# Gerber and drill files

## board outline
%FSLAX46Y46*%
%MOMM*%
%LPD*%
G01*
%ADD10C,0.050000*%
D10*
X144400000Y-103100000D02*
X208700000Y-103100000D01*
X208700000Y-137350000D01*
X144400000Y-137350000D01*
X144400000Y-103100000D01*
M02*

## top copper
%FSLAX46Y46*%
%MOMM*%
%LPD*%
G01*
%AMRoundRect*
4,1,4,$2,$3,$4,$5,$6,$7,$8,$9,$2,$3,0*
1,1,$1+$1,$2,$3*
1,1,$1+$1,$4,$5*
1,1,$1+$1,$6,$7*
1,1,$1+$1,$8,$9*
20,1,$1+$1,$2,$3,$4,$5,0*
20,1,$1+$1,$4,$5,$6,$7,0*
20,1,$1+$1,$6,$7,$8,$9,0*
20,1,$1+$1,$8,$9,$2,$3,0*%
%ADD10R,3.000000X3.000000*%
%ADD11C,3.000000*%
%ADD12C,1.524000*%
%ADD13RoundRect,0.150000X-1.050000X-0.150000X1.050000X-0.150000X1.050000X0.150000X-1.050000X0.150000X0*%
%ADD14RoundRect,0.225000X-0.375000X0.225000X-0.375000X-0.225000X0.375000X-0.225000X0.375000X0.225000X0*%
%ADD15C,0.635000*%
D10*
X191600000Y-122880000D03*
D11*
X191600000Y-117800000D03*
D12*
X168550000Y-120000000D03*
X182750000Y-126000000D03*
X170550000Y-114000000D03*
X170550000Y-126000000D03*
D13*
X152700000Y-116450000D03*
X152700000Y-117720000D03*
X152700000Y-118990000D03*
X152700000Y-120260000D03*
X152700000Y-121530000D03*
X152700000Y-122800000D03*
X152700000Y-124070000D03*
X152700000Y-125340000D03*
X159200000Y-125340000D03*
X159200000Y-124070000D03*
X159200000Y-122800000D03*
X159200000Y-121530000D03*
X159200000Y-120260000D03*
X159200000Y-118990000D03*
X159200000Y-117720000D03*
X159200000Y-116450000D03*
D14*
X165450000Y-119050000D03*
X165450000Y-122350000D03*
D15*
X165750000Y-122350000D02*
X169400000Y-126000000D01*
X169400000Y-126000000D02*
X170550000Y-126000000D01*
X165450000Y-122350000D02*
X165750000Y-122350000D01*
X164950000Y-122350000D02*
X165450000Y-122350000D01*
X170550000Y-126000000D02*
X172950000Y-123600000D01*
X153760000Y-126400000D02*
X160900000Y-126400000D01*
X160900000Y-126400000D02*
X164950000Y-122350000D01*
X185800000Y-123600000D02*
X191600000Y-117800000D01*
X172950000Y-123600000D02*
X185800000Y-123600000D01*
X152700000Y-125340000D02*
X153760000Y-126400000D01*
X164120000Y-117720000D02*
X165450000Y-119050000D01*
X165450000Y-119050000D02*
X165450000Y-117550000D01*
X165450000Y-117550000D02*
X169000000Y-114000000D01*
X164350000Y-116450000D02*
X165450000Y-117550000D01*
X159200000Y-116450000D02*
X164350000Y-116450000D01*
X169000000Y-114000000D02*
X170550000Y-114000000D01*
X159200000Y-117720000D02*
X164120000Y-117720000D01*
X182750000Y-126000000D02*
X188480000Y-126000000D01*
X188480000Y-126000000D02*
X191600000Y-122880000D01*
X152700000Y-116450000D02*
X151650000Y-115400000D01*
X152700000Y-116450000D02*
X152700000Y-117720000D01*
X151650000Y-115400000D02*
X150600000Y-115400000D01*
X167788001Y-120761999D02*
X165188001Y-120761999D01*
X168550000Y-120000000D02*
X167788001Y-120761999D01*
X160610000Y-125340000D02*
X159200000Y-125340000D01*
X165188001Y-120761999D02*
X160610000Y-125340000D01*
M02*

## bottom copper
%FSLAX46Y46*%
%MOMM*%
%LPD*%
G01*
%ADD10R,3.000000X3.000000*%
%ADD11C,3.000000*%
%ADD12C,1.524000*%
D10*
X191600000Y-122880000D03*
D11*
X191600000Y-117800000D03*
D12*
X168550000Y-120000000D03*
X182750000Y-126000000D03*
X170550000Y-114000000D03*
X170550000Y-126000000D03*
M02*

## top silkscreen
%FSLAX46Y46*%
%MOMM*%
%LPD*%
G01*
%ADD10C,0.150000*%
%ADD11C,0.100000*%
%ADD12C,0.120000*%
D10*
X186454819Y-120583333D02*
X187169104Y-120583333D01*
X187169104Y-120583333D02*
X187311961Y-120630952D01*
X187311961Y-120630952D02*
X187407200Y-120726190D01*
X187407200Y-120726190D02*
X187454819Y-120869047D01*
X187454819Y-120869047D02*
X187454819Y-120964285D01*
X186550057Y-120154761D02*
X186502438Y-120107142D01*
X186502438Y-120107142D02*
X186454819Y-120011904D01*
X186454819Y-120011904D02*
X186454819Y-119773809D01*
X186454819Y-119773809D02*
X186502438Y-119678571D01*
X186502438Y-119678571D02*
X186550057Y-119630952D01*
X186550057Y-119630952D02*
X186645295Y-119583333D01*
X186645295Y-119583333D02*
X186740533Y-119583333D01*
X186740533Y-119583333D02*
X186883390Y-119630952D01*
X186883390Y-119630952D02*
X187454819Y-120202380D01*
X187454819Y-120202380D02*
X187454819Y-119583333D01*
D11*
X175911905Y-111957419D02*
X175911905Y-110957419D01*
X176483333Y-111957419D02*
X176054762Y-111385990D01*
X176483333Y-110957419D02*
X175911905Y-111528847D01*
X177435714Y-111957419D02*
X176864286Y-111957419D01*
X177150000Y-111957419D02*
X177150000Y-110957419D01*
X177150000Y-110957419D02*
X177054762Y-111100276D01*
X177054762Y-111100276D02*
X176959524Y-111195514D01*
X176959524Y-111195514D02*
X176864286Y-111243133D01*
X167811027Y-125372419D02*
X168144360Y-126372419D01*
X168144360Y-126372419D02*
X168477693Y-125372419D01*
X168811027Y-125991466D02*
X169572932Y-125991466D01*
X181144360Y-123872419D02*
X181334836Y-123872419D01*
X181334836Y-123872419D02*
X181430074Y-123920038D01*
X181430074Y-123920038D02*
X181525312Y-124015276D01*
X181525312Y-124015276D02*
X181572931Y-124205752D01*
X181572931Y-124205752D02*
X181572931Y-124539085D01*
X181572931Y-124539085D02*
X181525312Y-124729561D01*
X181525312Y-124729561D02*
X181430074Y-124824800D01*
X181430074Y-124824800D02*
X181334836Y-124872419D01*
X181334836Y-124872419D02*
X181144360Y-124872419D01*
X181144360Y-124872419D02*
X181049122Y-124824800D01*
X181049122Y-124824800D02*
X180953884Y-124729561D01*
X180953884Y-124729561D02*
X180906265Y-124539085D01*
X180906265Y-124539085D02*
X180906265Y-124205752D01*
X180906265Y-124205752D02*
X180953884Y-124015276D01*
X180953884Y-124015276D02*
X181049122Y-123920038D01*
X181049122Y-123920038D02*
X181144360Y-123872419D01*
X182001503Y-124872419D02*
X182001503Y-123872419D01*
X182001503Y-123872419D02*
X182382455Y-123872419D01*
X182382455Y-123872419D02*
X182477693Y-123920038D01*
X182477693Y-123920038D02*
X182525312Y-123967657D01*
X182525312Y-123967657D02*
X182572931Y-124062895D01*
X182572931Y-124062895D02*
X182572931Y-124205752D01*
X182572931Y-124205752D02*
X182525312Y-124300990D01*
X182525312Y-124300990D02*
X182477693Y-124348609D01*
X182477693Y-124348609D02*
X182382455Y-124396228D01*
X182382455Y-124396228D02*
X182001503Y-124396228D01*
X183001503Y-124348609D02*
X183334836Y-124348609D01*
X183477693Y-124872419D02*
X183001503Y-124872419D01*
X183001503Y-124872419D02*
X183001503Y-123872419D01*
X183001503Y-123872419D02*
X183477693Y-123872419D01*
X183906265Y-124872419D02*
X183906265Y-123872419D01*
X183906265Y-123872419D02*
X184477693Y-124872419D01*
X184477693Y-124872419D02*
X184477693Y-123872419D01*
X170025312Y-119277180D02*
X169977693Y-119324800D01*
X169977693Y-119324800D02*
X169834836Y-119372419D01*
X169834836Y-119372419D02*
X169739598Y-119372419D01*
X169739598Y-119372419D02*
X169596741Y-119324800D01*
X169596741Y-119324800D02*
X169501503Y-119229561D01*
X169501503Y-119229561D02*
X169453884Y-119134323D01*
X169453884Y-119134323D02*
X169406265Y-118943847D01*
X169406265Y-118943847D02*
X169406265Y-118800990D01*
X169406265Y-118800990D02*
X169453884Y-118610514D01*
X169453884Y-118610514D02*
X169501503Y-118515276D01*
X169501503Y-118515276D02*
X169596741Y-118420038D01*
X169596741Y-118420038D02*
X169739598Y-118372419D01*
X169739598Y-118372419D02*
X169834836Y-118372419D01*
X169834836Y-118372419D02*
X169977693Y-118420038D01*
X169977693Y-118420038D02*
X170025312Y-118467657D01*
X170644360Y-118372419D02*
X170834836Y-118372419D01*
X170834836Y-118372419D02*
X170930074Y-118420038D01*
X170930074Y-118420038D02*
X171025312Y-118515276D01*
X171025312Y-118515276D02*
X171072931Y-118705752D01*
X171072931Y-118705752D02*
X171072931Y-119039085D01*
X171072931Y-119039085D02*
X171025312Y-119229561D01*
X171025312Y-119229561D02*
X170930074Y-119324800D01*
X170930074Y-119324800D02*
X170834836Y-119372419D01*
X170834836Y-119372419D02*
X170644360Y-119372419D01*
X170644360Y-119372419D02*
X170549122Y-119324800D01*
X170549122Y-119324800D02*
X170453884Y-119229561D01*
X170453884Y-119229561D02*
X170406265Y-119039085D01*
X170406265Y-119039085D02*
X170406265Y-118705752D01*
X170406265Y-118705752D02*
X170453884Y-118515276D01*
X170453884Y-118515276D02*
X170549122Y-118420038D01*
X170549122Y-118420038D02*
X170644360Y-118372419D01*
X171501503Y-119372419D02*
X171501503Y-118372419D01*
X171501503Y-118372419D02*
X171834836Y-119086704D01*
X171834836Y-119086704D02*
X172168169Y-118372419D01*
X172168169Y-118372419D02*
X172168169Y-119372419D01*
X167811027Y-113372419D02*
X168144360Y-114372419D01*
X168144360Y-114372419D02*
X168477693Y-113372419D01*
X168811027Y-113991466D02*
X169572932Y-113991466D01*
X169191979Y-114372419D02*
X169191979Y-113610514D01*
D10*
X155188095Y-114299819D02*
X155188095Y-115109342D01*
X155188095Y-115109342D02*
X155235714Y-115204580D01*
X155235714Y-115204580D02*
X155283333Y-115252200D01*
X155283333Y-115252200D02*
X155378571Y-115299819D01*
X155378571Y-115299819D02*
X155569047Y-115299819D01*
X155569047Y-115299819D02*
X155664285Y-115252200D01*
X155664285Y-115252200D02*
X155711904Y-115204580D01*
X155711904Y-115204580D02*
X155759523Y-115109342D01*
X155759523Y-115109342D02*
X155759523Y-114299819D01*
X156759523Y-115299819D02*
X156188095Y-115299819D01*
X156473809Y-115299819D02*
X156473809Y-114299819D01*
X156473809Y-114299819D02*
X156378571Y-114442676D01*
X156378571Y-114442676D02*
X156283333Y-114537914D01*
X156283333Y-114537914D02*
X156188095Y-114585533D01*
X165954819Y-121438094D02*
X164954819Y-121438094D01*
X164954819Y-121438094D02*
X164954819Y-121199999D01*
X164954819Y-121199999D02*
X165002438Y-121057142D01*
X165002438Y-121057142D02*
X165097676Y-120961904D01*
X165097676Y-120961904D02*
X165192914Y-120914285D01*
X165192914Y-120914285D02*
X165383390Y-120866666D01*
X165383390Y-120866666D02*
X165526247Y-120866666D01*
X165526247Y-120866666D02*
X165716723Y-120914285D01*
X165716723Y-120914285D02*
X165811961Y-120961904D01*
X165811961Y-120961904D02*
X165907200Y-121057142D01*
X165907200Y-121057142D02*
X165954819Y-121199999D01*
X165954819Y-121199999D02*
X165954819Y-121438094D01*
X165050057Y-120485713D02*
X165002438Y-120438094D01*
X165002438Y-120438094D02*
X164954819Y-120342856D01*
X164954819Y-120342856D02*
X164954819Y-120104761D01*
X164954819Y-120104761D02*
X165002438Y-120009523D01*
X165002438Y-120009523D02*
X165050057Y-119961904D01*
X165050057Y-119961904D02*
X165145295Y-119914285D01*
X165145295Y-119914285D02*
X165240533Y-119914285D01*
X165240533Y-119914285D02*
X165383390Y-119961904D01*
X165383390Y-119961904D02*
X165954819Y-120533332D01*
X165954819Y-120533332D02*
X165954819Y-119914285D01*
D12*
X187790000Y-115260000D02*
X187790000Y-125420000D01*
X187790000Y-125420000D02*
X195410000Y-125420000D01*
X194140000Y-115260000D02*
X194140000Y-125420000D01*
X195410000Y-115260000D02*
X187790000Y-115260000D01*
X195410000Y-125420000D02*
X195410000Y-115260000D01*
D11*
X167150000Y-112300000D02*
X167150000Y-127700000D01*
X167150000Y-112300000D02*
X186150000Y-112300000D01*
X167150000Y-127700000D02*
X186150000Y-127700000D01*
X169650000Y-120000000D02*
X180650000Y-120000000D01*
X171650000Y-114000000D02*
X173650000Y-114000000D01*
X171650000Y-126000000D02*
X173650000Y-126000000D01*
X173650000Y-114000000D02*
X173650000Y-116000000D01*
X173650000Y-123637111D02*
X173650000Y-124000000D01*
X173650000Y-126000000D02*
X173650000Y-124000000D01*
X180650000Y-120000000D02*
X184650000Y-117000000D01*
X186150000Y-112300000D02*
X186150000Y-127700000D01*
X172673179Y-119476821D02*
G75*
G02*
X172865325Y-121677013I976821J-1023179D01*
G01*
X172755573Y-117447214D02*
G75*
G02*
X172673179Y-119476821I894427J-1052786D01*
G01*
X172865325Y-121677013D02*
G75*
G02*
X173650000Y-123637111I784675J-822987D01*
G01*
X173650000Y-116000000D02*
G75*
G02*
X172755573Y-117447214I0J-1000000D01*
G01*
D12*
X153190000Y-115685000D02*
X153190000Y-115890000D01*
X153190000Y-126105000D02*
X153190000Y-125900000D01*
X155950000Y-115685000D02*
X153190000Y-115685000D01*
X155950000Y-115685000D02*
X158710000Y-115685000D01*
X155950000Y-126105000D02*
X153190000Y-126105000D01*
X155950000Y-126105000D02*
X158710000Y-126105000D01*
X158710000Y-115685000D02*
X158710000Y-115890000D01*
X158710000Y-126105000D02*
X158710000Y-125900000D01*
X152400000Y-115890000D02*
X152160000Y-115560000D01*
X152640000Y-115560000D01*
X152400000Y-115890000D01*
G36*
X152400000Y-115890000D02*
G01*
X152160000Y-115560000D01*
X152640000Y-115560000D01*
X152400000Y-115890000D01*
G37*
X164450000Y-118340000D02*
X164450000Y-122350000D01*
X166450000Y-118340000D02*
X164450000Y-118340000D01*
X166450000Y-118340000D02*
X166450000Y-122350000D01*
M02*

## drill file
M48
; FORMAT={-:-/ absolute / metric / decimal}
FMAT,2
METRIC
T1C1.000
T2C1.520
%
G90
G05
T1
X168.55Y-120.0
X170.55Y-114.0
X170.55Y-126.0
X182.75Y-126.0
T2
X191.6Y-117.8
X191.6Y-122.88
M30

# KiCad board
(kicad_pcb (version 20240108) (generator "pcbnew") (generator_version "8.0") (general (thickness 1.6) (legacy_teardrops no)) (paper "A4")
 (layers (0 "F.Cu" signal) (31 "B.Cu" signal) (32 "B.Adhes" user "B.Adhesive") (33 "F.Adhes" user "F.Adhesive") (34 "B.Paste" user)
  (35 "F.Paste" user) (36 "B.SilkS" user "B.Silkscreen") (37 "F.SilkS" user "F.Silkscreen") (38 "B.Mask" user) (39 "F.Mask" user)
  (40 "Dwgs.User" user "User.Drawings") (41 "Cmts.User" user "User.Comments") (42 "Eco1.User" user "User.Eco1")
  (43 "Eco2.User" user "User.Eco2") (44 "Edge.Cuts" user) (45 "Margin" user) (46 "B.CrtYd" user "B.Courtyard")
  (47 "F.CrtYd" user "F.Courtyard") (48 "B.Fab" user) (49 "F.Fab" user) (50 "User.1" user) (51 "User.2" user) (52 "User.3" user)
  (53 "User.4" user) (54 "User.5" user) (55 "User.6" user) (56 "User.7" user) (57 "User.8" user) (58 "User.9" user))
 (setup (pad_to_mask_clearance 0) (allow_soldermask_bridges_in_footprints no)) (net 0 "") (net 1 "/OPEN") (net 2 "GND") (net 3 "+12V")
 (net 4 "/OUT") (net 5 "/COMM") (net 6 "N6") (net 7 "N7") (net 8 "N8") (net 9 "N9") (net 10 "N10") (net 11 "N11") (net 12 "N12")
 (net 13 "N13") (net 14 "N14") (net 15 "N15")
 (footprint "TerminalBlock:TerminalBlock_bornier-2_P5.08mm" (layer "F.Cu") (at 191.6 122.88 90)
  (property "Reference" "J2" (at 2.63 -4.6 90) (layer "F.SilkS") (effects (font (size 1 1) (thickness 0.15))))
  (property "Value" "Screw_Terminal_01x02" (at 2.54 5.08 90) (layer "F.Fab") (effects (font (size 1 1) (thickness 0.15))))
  (fp_line (start 7.62 -3.81) (end -2.54 -3.81) (stroke (width 0.12) (type solid)) (layer "F.SilkS"))
  (fp_line (start -2.54 -3.81) (end -2.54 3.81) (stroke (width 0.12) (type solid)) (layer "F.SilkS"))
  (fp_line (start 7.62 2.54) (end -2.54 2.54) (stroke (width 0.12) (type solid)) (layer "F.SilkS"))
  (fp_line (start 7.62 3.81) (end 7.62 -3.81) (stroke (width 0.12) (type solid)) (layer "F.SilkS"))
  (fp_line (start -2.54 3.81) (end 7.62 3.81) (stroke (width 0.12) (type solid)) (layer "F.SilkS"))
  (pad "1" thru_hole rect (at 0 0 90) (size 3 3) (drill 1.52) (layers "*.Cu" "*.Mask") (remove_unused_layers no) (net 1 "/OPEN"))
  (pad "2" thru_hole circle (at 5.08 0 90) (size 3 3) (drill 1.52) (layers "*.Cu" "*.Mask") (remove_unused_layers no) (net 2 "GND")))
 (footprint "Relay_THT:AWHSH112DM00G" (layer "F.Cu") (at 176.65 120)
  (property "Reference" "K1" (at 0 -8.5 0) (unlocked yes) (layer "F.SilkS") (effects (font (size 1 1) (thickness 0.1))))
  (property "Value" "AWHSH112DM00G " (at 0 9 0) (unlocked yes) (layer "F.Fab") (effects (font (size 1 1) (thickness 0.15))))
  (fp_line (start -9.5 -7.7) (end -9.5 7.7) (stroke (width 0.1) (type default)) (layer "F.SilkS"))
  (fp_line (start -9.5 -7.7) (end 9.5 -7.7) (stroke (width 0.1) (type default)) (layer "F.SilkS"))
  (fp_line (start -9.5 7.7) (end 9.5 7.7) (stroke (width 0.1) (type default)) (layer "F.SilkS"))
  (fp_line (start -7 0) (end 4 0) (stroke (width 0.1) (type default)) (layer "F.SilkS"))
  (fp_line (start -5 -6) (end -3 -6) (stroke (width 0.1) (type default)) (layer "F.SilkS"))
  (fp_line (start -5 6) (end -3 6) (stroke (width 0.1) (type default)) (layer "F.SilkS"))
  (fp_line (start -3 -6) (end -3 -4) (stroke (width 0.1) (type default)) (layer "F.SilkS"))
  (fp_line (start -3 3.637111) (end -3 4) (stroke (width 0.1) (type default)) (layer "F.SilkS"))
  (fp_line (start -3 6) (end -3 4) (stroke (width 0.1) (type default)) (layer "F.SilkS"))
  (fp_line (start 4 0) (end 8 -3) (stroke (width 0.1) (type default)) (layer "F.SilkS"))
  (fp_line (start 9.5 -7.7) (end 9.5 7.7) (stroke (width 0.1) (type default)) (layer "F.SilkS"))
  (fp_arc (start -3.976821 -0.523179) (mid -1.59077 0.37693) (end -3.784675 1.677013) (stroke (width 0.1) (type default)) (layer "F.SilkS"))
  (fp_arc (start -3.894427 -2.552786) (mid -1.619704 -1.443966) (end -3.976821 -0.523179) (stroke (width 0.1) (type default))
   (layer "F.SilkS"))
  (fp_arc (start -3.784675 1.677013) (mid -1.944337 2.077392) (end -3 3.637111) (stroke (width 0.1) (type default)) (layer "F.SilkS"))
  (fp_arc (start -3 -4) (mid -2.149349 -2.474269) (end -3.894427 -2.552786) (stroke (width 0.1) (type default)) (layer "F.SilkS"))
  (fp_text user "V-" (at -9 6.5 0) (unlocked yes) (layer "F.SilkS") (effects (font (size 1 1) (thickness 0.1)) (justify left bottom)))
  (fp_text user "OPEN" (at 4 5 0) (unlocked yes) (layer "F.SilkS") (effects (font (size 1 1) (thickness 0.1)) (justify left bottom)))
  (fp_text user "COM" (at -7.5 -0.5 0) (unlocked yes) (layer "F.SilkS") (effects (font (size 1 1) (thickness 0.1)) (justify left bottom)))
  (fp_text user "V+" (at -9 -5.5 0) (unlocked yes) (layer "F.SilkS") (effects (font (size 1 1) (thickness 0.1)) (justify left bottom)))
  (pad "COM" thru_hole circle (at -8.1 0) (size 1.524 1.524) (drill 1) (layers "*.Cu" "*.Mask") (remove_unused_layers no) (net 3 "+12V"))
  (pad "OPEN" thru_hole circle (at 6.1 6) (size 1.524 1.524) (drill 1) (layers "*.Cu" "*.Mask") (remove_unused_layers no) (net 1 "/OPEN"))
  (pad "V+" thru_hole circle (at -6.1 -6) (size 1.524 1.524) (drill 1) (layers "*.Cu" "*.Mask") (remove_unused_layers no) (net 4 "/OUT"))
  (pad "V-" thru_hole circle (at -6.1 6) (size 1.524 1.524) (drill 1) (layers "*.Cu" "*.Mask") (remove_unused_layers no) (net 2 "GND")))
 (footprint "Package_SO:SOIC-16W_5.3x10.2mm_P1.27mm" (layer "F.Cu") (at 155.95 120.895)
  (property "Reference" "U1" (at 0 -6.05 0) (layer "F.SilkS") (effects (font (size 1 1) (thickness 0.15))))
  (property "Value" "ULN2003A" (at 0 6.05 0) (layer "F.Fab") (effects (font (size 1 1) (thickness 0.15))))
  (fp_line (start -2.76 -5.21) (end -2.76 -5.005) (stroke (width 0.12) (type solid)) (layer "F.SilkS"))
  (fp_line (start -2.76 5.21) (end -2.76 5.005) (stroke (width 0.12) (type solid)) (layer "F.SilkS"))
  (fp_line (start 0 -5.21) (end -2.76 -5.21) (stroke (width 0.12) (type solid)) (layer "F.SilkS"))
  (fp_line (start 0 -5.21) (end 2.76 -5.21) (stroke (width 0.12) (type solid)) (layer "F.SilkS"))
  (fp_line (start 0 5.21) (end -2.76 5.21) (stroke (width 0.12) (type solid)) (layer "F.SilkS"))
  (fp_line (start 0 5.21) (end 2.76 5.21) (stroke (width 0.12) (type solid)) (layer "F.SilkS"))
  (fp_line (start 2.76 -5.21) (end 2.76 -5.005) (stroke (width 0.12) (type solid)) (layer "F.SilkS"))
  (fp_line (start 2.76 5.21) (end 2.76 5.005) (stroke (width 0.12) (type solid)) (layer "F.SilkS"))
  (fp_poly
   (pts (xy -3.55 -5.005) (xy -3.79 -5.335) (xy -3.31 -5.335) (xy -3.55 -5.005)) (stroke (width 0.12) (type solid)) (fill solid)
   (layer "F.SilkS"))
  (pad "1" smd roundrect (at -3.25 -4.445) (size 2.4 0.6) (layers "F.Cu" "F.Paste" "F.Mask") (roundrect_rratio 0.25) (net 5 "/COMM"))
  (pad "2" smd roundrect (at -3.25 -3.175) (size 2.4 0.6) (layers "F.Cu" "F.Paste" "F.Mask") (roundrect_rratio 0.25) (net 5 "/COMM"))
  (pad "3" smd roundrect (at -3.25 -1.905) (size 2.4 0.6) (layers "F.Cu" "F.Paste" "F.Mask") (roundrect_rratio 0.25) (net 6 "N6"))
  (pad "4" smd roundrect (at -3.25 -0.635) (size 2.4 0.6) (layers "F.Cu" "F.Paste" "F.Mask") (roundrect_rratio 0.25) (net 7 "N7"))
  (pad "5" smd roundrect (at -3.25 0.635) (size 2.4 0.6) (layers "F.Cu" "F.Paste" "F.Mask") (roundrect_rratio 0.25) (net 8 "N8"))
  (pad "6" smd roundrect (at -3.25 1.905) (size 2.4 0.6) (layers "F.Cu" "F.Paste" "F.Mask") (roundrect_rratio 0.25) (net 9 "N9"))
  (pad "7" smd roundrect (at -3.25 3.175) (size 2.4 0.6) (layers "F.Cu" "F.Paste" "F.Mask") (roundrect_rratio 0.25) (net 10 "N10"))
  (pad "8" smd roundrect (at -3.25 4.445) (size 2.4 0.6) (layers "F.Cu" "F.Paste" "F.Mask") (roundrect_rratio 0.25) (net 2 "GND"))
  (pad "9" smd roundrect (at 3.25 4.445) (size 2.4 0.6) (layers "F.Cu" "F.Paste" "F.Mask") (roundrect_rratio 0.25) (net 3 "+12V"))
  (pad "10" smd roundrect (at 3.25 3.175) (size 2.4 0.6) (layers "F.Cu" "F.Paste" "F.Mask") (roundrect_rratio 0.25) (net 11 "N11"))
  (pad "11" smd roundrect (at 3.25 1.905) (size 2.4 0.6) (layers "F.Cu" "F.Paste" "F.Mask") (roundrect_rratio 0.25) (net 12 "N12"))
  (pad "12" smd roundrect (at 3.25 0.635) (size 2.4 0.6) (layers "F.Cu" "F.Paste" "F.Mask") (roundrect_rratio 0.25) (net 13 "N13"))
  (pad "13" smd roundrect (at 3.25 -0.635) (size 2.4 0.6) (layers "F.Cu" "F.Paste" "F.Mask") (roundrect_rratio 0.25) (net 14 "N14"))
  (pad "14" smd roundrect (at 3.25 -1.905) (size 2.4 0.6) (layers "F.Cu" "F.Paste" "F.Mask") (roundrect_rratio 0.25) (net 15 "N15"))
  (pad "15" smd roundrect (at 3.25 -3.175) (size 2.4 0.6) (layers "F.Cu" "F.Paste" "F.Mask") (roundrect_rratio 0.25) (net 4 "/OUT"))
  (pad "16" smd roundrect (at 3.25 -4.445) (size 2.4 0.6) (layers "F.Cu" "F.Paste" "F.Mask") (roundrect_rratio 0.25) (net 4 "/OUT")))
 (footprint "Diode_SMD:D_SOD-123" (layer "F.Cu") (at 165.45 120.7 -90)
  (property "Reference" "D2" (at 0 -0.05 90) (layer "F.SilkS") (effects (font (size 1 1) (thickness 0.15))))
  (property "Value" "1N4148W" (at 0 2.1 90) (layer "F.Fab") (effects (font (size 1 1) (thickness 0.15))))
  (fp_line (start -2.36 1) (end 1.65 1) (stroke (width 0.12) (type solid)) (layer "F.SilkS"))
  (fp_line (start -2.36 -1) (end -2.36 1) (stroke (width 0.12) (type solid)) (layer "F.SilkS"))
  (fp_line (start -2.36 -1) (end 1.65 -1) (stroke (width 0.12) (type solid)) (layer "F.SilkS"))
  (pad "1" smd roundrect (at -1.65 0 270) (size 0.9 1.2) (layers "F.Cu" "F.Paste" "F.Mask") (roundrect_rratio 0.25) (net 4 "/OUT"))
  (pad "2" smd roundrect (at 1.65 0 270) (size 0.9 1.2) (layers "F.Cu" "F.Paste" "F.Mask") (roundrect_rratio 0.25) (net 2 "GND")))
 (gr_rect (start 144.4 103.1) (end 208.7 137.35) (stroke (width 0.05) (type default)) (fill none) (layer "Edge.Cuts"))
 (segment (start 165.75 122.35) (end 169.4 126) (width 0.635) (layer "F.Cu") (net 2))
 (segment (start 169.4 126) (end 170.55 126) (width 0.635) (layer "F.Cu") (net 2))
 (segment (start 165.45 122.35) (end 165.75 122.35) (width 0.635) (layer "F.Cu") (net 2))
 (segment (start 164.95 122.35) (end 165.45 122.35) (width 0.635) (layer "F.Cu") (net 2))
 (segment (start 170.55 126) (end 172.95 123.6) (width 0.635) (layer "F.Cu") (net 2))
 (segment (start 153.76 126.4) (end 160.9 126.4) (width 0.635) (layer "F.Cu") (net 2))
 (segment (start 160.9 126.4) (end 164.95 122.35) (width 0.635) (layer "F.Cu") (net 2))
 (segment (start 185.8 123.6) (end 191.6 117.8) (width 0.635) (layer "F.Cu") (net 2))
 (segment (start 172.95 123.6) (end 185.8 123.6) (width 0.635) (layer "F.Cu") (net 2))
 (segment (start 152.7 125.34) (end 153.76 126.4) (width 0.635) (layer "F.Cu") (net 2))
 (segment (start 164.12 117.72) (end 165.45 119.05) (width 0.635) (layer "F.Cu") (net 4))
 (segment (start 165.45 119.05) (end 165.45 117.55) (width 0.635) (layer "F.Cu") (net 4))
 (segment (start 165.45 117.55) (end 169 114) (width 0.635) (layer "F.Cu") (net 4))
 (segment (start 164.35 116.45) (end 165.45 117.55) (width 0.635) (layer "F.Cu") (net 4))
 (segment (start 159.2 116.45) (end 164.35 116.45) (width 0.635) (layer "F.Cu") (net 4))
 (segment (start 169 114) (end 170.55 114) (width 0.635) (layer "F.Cu") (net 4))
 (segment (start 159.2 117.72) (end 164.12 117.72) (width 0.635) (layer "F.Cu") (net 4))
 (segment (start 182.75 126) (end 188.48 126) (width 0.635) (layer "F.Cu") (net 1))
 (segment (start 188.48 126) (end 191.6 122.88) (width 0.635) (layer "F.Cu") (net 1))
 (segment (start 152.7 116.45) (end 151.65 115.4) (width 0.635) (layer "F.Cu") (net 5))
 (segment (start 152.7 116.45) (end 152.7 117.72) (width 0.635) (layer "F.Cu") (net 5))
 (segment (start 151.65 115.4) (end 150.6 115.4) (width 0.635) (layer "F.Cu") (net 5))
 (segment (start 167.788001 120.761999) (end 165.188001 120.761999) (width 0.635) (layer "F.Cu") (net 3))
 (segment (start 168.55 120) (end 167.788001 120.761999) (width 0.635) (layer "F.Cu") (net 3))
 (segment (start 160.61 125.34) (end 159.2 125.34) (width 0.635) (layer "F.Cu") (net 3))
 (segment (start 165.188001 120.761999) (end 160.61 125.34) (width 0.635) (layer "F.Cu") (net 3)))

